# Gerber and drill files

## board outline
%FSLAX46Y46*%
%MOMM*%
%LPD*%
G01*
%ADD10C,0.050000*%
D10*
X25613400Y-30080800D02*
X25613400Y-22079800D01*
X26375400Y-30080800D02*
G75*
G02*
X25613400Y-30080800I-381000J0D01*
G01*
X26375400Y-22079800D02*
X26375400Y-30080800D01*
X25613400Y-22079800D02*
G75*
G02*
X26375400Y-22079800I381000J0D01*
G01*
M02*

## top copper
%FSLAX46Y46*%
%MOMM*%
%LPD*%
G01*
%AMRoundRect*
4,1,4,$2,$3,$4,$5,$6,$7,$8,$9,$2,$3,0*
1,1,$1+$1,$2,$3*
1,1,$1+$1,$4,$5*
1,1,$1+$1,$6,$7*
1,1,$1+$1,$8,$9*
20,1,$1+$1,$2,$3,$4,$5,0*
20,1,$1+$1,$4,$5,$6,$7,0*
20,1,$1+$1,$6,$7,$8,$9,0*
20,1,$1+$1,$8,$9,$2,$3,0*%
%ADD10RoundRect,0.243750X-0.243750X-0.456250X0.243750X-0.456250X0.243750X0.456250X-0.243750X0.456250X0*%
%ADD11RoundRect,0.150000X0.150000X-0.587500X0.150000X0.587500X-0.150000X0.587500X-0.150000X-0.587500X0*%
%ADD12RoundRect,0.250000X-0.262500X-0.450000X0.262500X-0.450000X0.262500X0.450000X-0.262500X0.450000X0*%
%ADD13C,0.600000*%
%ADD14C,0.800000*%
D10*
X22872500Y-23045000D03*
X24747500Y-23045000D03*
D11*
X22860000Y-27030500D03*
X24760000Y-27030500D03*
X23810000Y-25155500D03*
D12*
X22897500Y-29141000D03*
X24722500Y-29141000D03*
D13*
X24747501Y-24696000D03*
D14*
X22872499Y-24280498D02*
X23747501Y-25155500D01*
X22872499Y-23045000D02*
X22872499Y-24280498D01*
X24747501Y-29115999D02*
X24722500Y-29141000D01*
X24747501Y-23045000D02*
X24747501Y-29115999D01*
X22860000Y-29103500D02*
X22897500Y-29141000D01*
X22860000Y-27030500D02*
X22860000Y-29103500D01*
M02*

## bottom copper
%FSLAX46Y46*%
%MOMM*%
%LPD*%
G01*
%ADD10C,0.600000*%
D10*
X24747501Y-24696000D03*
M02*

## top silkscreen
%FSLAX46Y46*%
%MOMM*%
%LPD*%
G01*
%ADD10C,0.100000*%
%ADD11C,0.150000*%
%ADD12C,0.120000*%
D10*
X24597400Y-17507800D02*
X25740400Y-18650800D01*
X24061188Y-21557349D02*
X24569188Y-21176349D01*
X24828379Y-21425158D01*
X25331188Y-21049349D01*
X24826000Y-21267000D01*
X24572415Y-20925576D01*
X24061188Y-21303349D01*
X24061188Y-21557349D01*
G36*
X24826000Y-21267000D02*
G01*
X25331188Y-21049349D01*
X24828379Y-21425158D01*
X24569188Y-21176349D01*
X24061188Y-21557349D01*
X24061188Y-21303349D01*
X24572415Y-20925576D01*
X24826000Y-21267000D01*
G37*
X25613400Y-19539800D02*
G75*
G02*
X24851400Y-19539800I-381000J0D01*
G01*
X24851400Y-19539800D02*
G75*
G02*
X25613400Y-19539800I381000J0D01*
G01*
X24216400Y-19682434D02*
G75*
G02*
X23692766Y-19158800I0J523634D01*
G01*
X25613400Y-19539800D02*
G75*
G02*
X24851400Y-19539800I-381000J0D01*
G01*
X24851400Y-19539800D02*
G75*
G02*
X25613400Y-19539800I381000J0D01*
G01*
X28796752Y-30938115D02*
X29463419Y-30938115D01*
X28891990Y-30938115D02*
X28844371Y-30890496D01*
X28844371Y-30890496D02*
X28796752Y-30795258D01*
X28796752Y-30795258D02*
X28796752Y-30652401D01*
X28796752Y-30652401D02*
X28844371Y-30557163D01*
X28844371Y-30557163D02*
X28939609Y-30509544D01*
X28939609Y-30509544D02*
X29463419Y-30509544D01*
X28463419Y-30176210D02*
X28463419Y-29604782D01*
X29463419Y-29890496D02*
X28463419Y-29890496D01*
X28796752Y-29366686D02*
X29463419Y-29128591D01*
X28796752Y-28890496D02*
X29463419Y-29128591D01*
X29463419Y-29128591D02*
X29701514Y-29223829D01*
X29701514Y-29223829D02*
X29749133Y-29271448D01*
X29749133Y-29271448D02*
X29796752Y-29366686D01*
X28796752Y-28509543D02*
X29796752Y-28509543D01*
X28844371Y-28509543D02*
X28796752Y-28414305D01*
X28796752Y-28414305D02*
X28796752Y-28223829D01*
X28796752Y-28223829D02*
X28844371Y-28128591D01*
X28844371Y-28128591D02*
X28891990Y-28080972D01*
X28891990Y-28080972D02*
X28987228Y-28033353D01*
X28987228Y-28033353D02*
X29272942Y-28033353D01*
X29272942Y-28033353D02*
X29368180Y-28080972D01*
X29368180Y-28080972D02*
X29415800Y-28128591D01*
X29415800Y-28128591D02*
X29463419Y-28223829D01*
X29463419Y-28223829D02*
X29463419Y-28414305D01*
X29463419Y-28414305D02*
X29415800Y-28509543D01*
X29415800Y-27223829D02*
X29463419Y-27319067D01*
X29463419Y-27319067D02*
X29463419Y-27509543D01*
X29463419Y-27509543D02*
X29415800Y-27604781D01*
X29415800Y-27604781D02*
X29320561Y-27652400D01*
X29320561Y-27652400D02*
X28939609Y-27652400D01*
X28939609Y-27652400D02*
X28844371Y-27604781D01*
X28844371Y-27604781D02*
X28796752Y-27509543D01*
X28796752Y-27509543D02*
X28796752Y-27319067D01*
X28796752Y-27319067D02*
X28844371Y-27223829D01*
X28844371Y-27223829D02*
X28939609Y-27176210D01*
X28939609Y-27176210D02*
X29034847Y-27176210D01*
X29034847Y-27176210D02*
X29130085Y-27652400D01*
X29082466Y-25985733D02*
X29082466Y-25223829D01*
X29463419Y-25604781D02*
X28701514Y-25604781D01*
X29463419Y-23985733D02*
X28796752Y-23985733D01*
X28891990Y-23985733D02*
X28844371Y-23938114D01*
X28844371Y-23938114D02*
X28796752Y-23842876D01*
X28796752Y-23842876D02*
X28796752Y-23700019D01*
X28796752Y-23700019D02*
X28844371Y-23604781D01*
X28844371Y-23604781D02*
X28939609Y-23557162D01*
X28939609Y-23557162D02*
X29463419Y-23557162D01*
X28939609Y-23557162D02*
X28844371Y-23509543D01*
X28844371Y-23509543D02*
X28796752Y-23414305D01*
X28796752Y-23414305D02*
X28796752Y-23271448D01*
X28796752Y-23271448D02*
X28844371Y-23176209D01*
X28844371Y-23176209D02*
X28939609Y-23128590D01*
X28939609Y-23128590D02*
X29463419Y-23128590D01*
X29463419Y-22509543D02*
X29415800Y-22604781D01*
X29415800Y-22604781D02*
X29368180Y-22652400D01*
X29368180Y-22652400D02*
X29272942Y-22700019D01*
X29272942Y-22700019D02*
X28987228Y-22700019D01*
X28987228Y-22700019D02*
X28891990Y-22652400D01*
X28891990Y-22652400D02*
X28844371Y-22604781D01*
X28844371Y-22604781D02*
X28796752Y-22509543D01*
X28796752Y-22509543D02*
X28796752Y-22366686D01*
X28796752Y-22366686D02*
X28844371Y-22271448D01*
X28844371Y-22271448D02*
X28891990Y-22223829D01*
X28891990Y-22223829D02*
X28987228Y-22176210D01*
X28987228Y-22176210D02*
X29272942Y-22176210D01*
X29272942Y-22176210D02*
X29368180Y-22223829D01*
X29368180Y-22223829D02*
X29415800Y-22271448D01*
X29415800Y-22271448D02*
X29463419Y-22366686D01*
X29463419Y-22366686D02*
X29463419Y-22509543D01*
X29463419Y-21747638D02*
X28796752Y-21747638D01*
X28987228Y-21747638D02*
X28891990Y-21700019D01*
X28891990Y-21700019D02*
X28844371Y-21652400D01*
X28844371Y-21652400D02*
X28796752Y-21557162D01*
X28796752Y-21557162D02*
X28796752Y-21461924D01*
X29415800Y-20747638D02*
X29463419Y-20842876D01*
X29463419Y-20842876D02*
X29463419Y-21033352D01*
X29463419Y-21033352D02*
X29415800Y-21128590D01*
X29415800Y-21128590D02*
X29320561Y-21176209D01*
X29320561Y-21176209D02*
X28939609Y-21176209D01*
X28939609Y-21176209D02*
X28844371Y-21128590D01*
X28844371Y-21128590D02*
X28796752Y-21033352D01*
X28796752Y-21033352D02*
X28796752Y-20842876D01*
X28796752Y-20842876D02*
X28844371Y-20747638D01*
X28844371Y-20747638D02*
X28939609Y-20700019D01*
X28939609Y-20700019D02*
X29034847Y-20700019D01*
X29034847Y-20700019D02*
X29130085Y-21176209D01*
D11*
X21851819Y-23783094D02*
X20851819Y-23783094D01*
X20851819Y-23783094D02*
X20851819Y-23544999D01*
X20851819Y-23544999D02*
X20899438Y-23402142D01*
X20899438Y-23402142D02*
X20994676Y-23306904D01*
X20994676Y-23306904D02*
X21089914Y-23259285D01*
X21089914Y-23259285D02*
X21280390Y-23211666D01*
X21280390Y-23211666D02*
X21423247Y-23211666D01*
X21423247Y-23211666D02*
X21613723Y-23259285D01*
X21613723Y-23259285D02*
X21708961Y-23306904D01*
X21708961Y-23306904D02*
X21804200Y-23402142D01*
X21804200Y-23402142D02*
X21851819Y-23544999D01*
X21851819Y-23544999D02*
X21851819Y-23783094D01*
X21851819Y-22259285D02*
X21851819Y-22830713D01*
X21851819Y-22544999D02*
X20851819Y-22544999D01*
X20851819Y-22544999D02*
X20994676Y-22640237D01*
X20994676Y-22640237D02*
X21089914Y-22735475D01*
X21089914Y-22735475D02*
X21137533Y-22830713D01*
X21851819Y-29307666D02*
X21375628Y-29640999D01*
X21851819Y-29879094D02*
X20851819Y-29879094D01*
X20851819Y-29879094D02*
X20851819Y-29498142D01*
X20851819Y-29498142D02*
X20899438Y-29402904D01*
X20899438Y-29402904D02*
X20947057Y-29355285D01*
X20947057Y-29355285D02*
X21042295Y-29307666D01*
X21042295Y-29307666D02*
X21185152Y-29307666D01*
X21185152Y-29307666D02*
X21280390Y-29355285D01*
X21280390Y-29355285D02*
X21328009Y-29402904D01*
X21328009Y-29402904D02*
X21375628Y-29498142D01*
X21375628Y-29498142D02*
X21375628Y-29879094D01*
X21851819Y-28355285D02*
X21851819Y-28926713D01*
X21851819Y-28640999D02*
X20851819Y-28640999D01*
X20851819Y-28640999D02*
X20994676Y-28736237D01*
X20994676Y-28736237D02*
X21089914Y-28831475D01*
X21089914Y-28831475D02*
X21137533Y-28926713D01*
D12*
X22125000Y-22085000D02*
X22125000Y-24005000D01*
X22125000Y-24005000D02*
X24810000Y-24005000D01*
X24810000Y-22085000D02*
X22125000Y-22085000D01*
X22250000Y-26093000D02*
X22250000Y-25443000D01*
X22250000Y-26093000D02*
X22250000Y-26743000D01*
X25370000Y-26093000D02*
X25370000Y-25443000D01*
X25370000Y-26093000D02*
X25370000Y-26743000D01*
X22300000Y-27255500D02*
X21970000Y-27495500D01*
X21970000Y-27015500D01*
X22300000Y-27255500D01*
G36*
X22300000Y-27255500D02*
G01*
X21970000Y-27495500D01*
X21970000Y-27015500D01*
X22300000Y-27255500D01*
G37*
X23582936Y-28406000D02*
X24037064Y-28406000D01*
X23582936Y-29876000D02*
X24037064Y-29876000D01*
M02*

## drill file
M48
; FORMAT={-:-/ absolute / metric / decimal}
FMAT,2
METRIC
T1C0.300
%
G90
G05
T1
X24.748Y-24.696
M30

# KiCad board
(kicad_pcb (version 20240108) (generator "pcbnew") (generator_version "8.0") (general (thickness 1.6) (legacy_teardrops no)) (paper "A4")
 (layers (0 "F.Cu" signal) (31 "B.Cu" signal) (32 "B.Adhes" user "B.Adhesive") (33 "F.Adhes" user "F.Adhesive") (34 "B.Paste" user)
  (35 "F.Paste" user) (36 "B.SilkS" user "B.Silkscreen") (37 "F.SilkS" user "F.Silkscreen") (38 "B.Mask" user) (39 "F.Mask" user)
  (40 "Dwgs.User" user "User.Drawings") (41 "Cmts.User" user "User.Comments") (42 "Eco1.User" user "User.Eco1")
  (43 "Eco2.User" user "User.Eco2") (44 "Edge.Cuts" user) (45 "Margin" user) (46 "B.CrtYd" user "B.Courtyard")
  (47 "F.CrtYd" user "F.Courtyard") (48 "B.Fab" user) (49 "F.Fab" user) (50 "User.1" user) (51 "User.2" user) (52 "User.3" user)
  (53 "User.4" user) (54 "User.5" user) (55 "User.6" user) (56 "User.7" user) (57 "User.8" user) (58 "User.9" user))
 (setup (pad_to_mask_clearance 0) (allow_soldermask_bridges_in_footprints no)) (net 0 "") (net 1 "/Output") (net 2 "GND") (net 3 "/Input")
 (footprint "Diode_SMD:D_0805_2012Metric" (layer "F.Cu") (at 23.81 23.045)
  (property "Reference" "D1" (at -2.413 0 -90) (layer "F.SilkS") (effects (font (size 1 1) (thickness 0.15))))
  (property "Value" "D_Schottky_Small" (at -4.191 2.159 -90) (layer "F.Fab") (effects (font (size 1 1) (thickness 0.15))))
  (fp_line (start -1.685 -0.96) (end -1.685 0.96) (stroke (width 0.12) (type solid)) (layer "F.SilkS"))
  (fp_line (start -1.685 0.96) (end 1 0.96) (stroke (width 0.12) (type solid)) (layer "F.SilkS"))
  (fp_line (start 1 -0.96) (end -1.685 -0.96) (stroke (width 0.12) (type solid)) (layer "F.SilkS"))
  (pad "1" smd roundrect (at -0.9375 0) (size 0.975 1.4) (layers "F.Cu" "F.Paste" "F.Mask") (roundrect_rratio 0.25) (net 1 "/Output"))
  (pad "2" smd roundrect (at 0.9375 0) (size 0.975 1.4) (layers "F.Cu" "F.Paste" "F.Mask") (roundrect_rratio 0.25) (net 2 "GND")))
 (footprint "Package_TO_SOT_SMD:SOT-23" (layer "F.Cu") (at 23.81 26.093 90)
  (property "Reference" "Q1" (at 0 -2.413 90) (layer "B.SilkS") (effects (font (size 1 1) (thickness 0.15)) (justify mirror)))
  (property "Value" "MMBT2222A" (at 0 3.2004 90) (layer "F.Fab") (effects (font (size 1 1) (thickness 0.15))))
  (fp_line (start 0 -1.56) (end 0.65 -1.56) (stroke (width 0.12) (type solid)) (layer "F.SilkS"))
  (fp_line (start 0 -1.56) (end -0.65 -1.56) (stroke (width 0.12) (type solid)) (layer "F.SilkS"))
  (fp_line (start 0 1.56) (end 0.65 1.56) (stroke (width 0.12) (type solid)) (layer "F.SilkS"))
  (fp_line (start 0 1.56) (end -0.65 1.56) (stroke (width 0.12) (type solid)) (layer "F.SilkS"))
  (fp_poly
   (pts (xy -1.1625 -1.51) (xy -1.4025 -1.84) (xy -0.9225 -1.84) (xy -1.1625 -1.51)) (stroke (width 0.12) (type solid)) (fill solid)
   (layer "F.SilkS"))
  (pad "1" smd roundrect (at -0.9375 -0.95 90) (size 1.475 0.6) (layers "F.Cu" "F.Paste" "F.Mask") (roundrect_rratio 0.25) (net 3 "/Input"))
  (pad "2" smd roundrect (at -0.9375 0.95 90) (size 1.475 0.6) (layers "F.Cu" "F.Paste" "F.Mask") (roundrect_rratio 0.25) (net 2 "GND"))
  (pad "3" smd roundrect (at 0.9375 0 90) (size 1.475 0.6) (layers "F.Cu" "F.Paste" "F.Mask") (roundrect_rratio 0.25) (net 1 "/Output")))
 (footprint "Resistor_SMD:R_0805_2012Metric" (layer "F.Cu") (at 23.81 29.141)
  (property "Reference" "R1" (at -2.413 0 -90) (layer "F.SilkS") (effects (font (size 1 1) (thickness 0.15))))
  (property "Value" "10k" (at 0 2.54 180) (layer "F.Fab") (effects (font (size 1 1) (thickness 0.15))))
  (fp_line (start -0.227064 -0.735) (end 0.227064 -0.735) (stroke (width 0.12) (type solid)) (layer "F.SilkS"))
  (fp_line (start -0.227064 0.735) (end 0.227064 0.735) (stroke (width 0.12) (type solid)) (layer "F.SilkS"))
  (pad "1" smd roundrect (at -0.9125 0) (size 1.025 1.4) (layers "F.Cu" "F.Paste" "F.Mask") (roundrect_rratio 0.243902) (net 3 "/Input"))
  (pad "2" smd roundrect (at 0.9125 0) (size 1.025 1.4) (layers "F.Cu" "F.Paste" "F.Mask") (roundrect_rratio 0.243902) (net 2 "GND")))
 (gr_line (start 24.5974 17.5078) (end 25.7404 18.6508) (stroke (width 0.1) (type default)) (layer "F.SilkS"))
 (gr_poly
  (pts (xy 24.061188 21.557349) (xy 24.569188 21.176349) (xy 24.828379 21.425158) (xy 25.331188 21.049349) (xy 24.826 21.267)
   (xy 24.572415 20.925576) (xy 24.061188 21.303349))
  (stroke (width 0.1) (type solid)) (fill solid) (layer "F.SilkS"))
 (gr_circle (center 25.2324 19.5398) (end 24.8514 19.5398) (stroke (width 0.1) (type default)) (fill none) (layer "F.SilkS"))
 (gr_arc (start 24.2164 19.682434) (mid 23.846135 19.529065) (end 23.692766 19.1588) (stroke (width 0.1) (type default)) (layer "F.SilkS"))
 (gr_circle (center 25.2324 19.5398) (end 24.8514 19.5398) (stroke (width 0.1) (type default)) (fill none) (layer "F.SilkS"))
 (gr_line (start 25.6134 30.0808) (end 25.6134 22.0798) (stroke (width 0.05) (type default)) (layer "Edge.Cuts"))
 (gr_arc (start 26.3754 30.0808) (mid 25.9944 30.4618) (end 25.6134 30.0808) (stroke (width 0.05) (type default)) (layer "Edge.Cuts"))
 (gr_line (start 26.3754 22.0798) (end 26.3754 30.0808) (stroke (width 0.05) (type default)) (layer "Edge.Cuts"))
 (gr_arc (start 25.6134 22.0798) (mid 25.9944 21.6988) (end 26.3754 22.0798) (stroke (width 0.05) (type default)) (layer "Edge.Cuts"))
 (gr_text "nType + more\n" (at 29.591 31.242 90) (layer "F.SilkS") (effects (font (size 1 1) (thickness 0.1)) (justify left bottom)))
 (segment (start 22.872499 24.280498) (end 23.747501 25.1555) (width 0.8) (layer "F.Cu") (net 1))
 (segment (start 22.872499 23.045) (end 22.872499 24.280498) (width 0.8) (layer "F.Cu") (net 1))
 (segment (start 24.747501 29.115999) (end 24.7225 29.141) (width 0.8) (layer "F.Cu") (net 2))
 (segment (start 24.747501 23.045) (end 24.747501 29.115999) (width 0.8) (layer "F.Cu") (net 2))
 (via (at 24.747501 24.696) (size 0.6) (drill 0.3) (layers "F.Cu" "B.Cu") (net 2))
 (segment (start 22.86 29.1035) (end 22.8975 29.141) (width 0.8) (layer "F.Cu") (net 3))
 (segment (start 22.86 27.0305) (end 22.86 29.1035) (width 0.8) (layer "F.Cu") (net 3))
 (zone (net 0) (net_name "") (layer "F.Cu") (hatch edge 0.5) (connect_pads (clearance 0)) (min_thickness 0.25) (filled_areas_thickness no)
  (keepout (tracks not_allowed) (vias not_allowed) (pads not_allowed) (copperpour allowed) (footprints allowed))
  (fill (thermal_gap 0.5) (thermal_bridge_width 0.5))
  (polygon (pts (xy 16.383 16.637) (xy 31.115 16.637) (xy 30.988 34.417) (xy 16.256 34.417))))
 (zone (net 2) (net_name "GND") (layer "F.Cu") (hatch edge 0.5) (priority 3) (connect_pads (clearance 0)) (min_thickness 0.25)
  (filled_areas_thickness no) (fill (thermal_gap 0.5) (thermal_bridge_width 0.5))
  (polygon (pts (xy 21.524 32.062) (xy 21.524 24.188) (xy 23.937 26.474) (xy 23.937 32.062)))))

